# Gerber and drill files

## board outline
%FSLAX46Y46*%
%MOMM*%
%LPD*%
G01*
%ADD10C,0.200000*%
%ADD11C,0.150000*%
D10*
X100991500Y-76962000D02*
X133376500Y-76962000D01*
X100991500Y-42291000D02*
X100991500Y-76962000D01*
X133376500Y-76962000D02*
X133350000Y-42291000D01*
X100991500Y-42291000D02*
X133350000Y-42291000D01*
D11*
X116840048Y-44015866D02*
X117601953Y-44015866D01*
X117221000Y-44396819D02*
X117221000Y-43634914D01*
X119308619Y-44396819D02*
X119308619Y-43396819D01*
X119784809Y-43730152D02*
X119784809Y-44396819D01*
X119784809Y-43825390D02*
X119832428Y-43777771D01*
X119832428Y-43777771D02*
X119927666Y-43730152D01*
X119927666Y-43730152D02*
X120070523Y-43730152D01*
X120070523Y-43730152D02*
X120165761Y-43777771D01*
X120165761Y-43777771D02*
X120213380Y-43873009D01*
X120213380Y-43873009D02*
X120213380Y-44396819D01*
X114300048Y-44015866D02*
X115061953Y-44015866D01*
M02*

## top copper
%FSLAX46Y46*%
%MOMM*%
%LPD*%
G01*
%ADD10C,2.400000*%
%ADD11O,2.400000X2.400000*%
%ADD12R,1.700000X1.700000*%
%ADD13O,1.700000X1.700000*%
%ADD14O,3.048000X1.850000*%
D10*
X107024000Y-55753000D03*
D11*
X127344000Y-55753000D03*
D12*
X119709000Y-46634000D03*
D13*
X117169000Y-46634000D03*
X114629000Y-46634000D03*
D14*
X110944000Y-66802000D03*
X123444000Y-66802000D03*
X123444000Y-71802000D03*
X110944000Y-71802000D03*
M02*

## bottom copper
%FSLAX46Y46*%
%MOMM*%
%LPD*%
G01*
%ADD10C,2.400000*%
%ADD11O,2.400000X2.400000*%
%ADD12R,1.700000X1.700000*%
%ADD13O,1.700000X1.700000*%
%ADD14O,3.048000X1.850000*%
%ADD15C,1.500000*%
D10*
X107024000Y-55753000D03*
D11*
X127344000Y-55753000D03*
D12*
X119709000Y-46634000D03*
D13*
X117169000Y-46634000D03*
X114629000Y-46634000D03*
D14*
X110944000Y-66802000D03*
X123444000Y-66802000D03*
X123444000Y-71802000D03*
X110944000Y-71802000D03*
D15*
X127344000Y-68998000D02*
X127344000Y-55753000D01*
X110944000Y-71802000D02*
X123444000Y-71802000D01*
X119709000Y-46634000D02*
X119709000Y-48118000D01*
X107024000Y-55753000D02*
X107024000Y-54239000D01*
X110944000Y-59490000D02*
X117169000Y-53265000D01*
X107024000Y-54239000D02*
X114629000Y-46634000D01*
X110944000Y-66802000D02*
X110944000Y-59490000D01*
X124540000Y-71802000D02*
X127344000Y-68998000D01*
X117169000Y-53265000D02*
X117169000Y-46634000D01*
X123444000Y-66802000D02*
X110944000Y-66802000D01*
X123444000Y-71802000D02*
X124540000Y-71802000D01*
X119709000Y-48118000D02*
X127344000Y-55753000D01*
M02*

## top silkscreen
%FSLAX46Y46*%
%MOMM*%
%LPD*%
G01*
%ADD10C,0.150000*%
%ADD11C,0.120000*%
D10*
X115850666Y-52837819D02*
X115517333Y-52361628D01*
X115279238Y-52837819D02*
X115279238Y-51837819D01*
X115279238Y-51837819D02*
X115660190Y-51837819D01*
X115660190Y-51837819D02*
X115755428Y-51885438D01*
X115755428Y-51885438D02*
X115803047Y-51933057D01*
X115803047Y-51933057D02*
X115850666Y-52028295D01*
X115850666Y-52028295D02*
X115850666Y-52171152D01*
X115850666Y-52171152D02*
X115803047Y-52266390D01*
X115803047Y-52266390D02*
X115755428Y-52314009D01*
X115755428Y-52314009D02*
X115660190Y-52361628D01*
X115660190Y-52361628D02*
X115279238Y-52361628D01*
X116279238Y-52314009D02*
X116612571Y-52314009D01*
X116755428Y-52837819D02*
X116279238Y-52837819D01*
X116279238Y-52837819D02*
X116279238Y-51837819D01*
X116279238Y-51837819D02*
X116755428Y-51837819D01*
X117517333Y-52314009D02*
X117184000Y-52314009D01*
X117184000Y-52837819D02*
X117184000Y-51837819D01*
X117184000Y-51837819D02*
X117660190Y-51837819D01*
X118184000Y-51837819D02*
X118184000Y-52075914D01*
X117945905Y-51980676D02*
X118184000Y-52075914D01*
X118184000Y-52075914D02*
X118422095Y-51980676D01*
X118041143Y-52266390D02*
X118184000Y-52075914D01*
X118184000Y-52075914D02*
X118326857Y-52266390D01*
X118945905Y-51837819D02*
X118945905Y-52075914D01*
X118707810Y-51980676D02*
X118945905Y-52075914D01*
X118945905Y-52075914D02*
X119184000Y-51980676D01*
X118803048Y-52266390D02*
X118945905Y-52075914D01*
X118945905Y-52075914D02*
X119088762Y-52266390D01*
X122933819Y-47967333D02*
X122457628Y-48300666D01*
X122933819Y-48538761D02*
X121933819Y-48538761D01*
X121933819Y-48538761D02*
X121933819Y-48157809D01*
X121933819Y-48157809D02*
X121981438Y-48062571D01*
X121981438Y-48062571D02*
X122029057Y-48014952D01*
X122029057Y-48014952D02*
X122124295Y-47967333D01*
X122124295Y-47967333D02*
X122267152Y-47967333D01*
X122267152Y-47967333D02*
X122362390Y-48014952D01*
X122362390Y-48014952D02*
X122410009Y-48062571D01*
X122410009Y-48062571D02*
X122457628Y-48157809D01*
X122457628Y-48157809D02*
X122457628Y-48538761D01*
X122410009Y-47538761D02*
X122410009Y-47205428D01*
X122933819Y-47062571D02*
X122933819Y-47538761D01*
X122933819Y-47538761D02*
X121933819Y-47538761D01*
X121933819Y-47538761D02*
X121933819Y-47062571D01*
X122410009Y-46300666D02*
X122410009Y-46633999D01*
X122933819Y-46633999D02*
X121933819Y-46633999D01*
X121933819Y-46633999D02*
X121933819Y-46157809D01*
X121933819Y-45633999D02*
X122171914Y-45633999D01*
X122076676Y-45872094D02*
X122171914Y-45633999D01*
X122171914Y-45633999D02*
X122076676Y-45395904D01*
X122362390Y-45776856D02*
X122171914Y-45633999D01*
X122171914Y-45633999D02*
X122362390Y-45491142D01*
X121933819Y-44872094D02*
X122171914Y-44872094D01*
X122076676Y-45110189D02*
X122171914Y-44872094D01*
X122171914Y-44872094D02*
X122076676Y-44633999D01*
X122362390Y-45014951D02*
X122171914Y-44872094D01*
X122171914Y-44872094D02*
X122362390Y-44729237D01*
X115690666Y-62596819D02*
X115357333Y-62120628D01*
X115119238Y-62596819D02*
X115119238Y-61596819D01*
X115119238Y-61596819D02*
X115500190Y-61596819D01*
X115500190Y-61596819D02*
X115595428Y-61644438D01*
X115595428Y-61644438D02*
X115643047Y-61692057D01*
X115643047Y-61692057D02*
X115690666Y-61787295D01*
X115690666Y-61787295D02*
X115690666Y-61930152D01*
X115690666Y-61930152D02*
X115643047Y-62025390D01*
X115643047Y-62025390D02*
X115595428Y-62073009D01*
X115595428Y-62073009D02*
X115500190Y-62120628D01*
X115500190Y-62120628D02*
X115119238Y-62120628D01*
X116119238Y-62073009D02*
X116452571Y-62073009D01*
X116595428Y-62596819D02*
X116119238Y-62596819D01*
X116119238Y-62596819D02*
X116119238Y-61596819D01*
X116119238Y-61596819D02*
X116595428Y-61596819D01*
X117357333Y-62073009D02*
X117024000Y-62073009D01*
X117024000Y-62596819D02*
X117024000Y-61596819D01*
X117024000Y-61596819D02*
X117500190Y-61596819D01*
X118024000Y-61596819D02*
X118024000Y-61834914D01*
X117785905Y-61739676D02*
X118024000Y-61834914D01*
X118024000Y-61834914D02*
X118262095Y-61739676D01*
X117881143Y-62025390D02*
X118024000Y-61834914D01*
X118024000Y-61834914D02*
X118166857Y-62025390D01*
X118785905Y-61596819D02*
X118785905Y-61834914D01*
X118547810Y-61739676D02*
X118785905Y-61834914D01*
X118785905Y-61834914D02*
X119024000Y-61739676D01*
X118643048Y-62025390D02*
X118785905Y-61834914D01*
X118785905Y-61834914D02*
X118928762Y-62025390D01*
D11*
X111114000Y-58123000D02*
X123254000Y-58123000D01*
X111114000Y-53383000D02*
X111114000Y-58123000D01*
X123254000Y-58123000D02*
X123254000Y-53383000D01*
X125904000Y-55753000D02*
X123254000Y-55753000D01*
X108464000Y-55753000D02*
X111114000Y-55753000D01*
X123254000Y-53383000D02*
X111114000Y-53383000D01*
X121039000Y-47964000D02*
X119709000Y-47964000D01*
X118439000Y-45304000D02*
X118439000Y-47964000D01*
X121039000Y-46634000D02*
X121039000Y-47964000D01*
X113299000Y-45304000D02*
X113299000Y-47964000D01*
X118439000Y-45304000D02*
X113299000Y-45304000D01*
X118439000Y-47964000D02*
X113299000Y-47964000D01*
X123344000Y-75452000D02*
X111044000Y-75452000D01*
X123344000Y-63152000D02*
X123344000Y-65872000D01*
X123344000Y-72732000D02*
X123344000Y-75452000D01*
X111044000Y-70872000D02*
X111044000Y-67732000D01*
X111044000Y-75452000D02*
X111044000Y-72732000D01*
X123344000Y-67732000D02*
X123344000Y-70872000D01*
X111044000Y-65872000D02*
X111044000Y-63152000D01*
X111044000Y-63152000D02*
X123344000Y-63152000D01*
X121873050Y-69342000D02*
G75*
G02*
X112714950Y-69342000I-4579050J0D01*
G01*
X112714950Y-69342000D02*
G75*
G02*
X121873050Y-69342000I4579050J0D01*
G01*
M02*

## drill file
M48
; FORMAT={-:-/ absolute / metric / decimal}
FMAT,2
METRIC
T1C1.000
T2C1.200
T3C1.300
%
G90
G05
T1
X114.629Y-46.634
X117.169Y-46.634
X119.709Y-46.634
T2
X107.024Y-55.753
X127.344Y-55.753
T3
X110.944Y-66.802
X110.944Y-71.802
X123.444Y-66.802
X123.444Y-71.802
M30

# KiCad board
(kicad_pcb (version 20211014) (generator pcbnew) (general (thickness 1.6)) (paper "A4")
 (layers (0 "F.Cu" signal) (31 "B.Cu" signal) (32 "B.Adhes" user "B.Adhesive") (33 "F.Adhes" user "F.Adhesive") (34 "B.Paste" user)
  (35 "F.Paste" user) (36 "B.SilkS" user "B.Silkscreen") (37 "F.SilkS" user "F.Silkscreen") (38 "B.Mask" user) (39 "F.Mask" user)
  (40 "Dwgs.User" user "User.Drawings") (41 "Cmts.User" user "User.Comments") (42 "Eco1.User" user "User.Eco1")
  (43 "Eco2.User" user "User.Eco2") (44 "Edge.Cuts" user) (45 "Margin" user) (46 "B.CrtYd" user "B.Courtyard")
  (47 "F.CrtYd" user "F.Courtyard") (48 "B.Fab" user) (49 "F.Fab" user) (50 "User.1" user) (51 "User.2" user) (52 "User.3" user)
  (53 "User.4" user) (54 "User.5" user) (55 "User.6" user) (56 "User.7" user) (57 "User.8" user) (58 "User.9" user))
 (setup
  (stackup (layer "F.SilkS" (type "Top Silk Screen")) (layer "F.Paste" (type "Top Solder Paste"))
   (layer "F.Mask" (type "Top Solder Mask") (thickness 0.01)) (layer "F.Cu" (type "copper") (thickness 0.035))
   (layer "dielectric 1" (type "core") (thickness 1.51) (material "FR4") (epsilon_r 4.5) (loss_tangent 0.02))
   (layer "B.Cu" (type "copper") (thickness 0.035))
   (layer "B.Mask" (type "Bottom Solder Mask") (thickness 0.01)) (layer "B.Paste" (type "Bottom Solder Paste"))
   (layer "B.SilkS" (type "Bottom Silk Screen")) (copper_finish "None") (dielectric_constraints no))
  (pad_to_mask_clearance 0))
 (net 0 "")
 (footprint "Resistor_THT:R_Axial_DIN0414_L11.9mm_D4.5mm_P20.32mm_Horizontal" (layer "F.Cu") (at 107.024 55.753)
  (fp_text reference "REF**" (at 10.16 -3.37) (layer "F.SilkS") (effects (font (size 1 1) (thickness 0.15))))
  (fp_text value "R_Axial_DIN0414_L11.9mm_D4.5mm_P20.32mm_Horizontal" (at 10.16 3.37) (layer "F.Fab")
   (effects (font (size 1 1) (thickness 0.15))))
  (fp_line (start 4.09 2.37) (end 16.23 2.37) (layer "F.SilkS") (width 0.12))
  (fp_line (start 4.09 -2.37) (end 4.09 2.37) (layer "F.SilkS") (width 0.12))
  (fp_line (start 16.23 2.37) (end 16.23 -2.37) (layer "F.SilkS") (width 0.12))
  (fp_line (start 18.88 0) (end 16.23 0) (layer "F.SilkS") (width 0.12))
  (fp_line (start 1.44 0) (end 4.09 0) (layer "F.SilkS") (width 0.12))
  (fp_line (start 16.23 -2.37) (end 4.09 -2.37) (layer "F.SilkS") (width 0.12))
  (pad "1" thru_hole circle (at 0 0) (size 2.4 2.4) (drill 1.2) (layers *.Cu *.Mask))
  (pad "2" thru_hole oval (at 20.32 0) (size 2.4 2.4) (drill 1.2) (layers *.Cu *.Mask)))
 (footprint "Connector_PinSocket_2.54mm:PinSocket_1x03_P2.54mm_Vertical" (layer "F.Cu") (at 119.709 46.634 -90)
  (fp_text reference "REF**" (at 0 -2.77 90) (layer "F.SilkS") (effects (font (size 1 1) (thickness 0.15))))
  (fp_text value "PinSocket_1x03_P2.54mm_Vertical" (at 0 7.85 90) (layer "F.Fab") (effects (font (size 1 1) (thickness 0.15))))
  (fp_line (start 1.33 -1.33) (end 1.33 0) (layer "F.SilkS") (width 0.12))
  (fp_line (start -1.33 1.27) (end 1.33 1.27) (layer "F.SilkS") (width 0.12))
  (fp_line (start 0 -1.33) (end 1.33 -1.33) (layer "F.SilkS") (width 0.12))
  (fp_line (start -1.33 6.41) (end 1.33 6.41) (layer "F.SilkS") (width 0.12))
  (fp_line (start -1.33 1.27) (end -1.33 6.41) (layer "F.SilkS") (width 0.12))
  (fp_line (start 1.33 1.27) (end 1.33 6.41) (layer "F.SilkS") (width 0.12))
  (pad "1" thru_hole rect (at 0 0 270) (size 1.7 1.7) (drill 1) (layers *.Cu *.Mask))
  (pad "2" thru_hole oval (at 0 2.54 270) (size 1.7 1.7) (drill 1) (layers *.Cu *.Mask))
  (pad "3" thru_hole oval (at 0 5.08 270) (size 1.7 1.7) (drill 1) (layers *.Cu *.Mask)))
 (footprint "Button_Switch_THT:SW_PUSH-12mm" (layer "F.Cu") (at 110.944 66.802)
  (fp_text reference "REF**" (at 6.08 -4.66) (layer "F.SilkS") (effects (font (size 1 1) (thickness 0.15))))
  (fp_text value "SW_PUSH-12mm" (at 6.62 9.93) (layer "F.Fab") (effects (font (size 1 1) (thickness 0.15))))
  (fp_line (start 12.4 8.65) (end 0.1 8.65) (layer "F.SilkS") (width 0.12))
  (fp_line (start 12.4 -3.65) (end 12.4 -0.93) (layer "F.SilkS") (width 0.12))
  (fp_line (start 12.4 5.93) (end 12.4 8.65) (layer "F.SilkS") (width 0.12))
  (fp_line (start 0.1 4.07) (end 0.1 0.93) (layer "F.SilkS") (width 0.12))
  (fp_line (start 0.1 8.65) (end 0.1 5.93) (layer "F.SilkS") (width 0.12))
  (fp_line (start 12.4 0.93) (end 12.4 4.07) (layer "F.SilkS") (width 0.12))
  (fp_line (start 0.1 -0.93) (end 0.1 -3.65) (layer "F.SilkS") (width 0.12))
  (fp_line (start 0.1 -3.65) (end 12.4 -3.65) (layer "F.SilkS") (width 0.12))
  (fp_circle (center 6.35 2.54) (end 10.16 5.08) (layer "F.SilkS") (width 0.12) (fill none))
  (pad "1" thru_hole oval (at 0 0) (size 3.048 1.85) (drill 1.3) (layers *.Cu *.Mask))
  (pad "1" thru_hole oval (at 12.5 0) (size 3.048 1.85) (drill 1.3) (layers *.Cu *.Mask))
  (pad "2" thru_hole oval (at 12.5 5) (size 3.048 1.85) (drill 1.3) (layers *.Cu *.Mask))
  (pad "2" thru_hole oval (at 0 5) (size 3.048 1.85) (drill 1.3) (layers *.Cu *.Mask)))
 (gr_line (start 100.9915 76.962) (end 133.3765 76.962) (layer "Edge.Cuts") (width 0.2))
 (gr_line (start 100.9915 42.291) (end 100.9915 76.962) (layer "Edge.Cuts") (width 0.2))
 (gr_line (start 133.3765 76.962) (end 133.35 42.291) (layer "Edge.Cuts") (width 0.2))
 (gr_line (start 100.9915 42.291) (end 133.35 42.291) (layer "Edge.Cuts") (width 0.2))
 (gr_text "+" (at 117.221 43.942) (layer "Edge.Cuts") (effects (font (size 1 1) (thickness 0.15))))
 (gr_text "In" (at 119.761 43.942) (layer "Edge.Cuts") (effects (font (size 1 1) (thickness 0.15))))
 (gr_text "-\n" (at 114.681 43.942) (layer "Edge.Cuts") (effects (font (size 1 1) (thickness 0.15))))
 (segment (start 127.344 68.998) (end 127.344 55.753) (width 1.5) (layer "B.Cu") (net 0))
 (segment (start 110.944 71.802) (end 123.444 71.802) (width 1.5) (layer "B.Cu") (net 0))
 (segment (start 119.709 46.634) (end 119.709 48.118) (width 1.5) (layer "B.Cu") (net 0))
 (segment (start 107.024 55.753) (end 107.024 54.239) (width 1.5) (layer "B.Cu") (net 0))
 (segment (start 110.944 59.49) (end 117.169 53.265) (width 1.5) (layer "B.Cu") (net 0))
 (segment (start 107.024 54.239) (end 114.629 46.634) (width 1.5) (layer "B.Cu") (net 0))
 (segment (start 110.944 66.802) (end 110.944 59.49) (width 1.5) (layer "B.Cu") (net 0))
 (segment (start 124.54 71.802) (end 127.344 68.998) (width 1.5) (layer "B.Cu") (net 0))
 (segment (start 117.169 53.265) (end 117.169 46.634) (width 1.5) (layer "B.Cu") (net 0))
 (segment (start 123.444 66.802) (end 110.944 66.802) (width 1.5) (layer "B.Cu") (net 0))
 (segment (start 123.444 71.802) (end 124.54 71.802) (width 1.5) (layer "B.Cu") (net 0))
 (segment (start 119.709 48.118) (end 127.344 55.753) (width 1.5) (layer "B.Cu") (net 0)))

